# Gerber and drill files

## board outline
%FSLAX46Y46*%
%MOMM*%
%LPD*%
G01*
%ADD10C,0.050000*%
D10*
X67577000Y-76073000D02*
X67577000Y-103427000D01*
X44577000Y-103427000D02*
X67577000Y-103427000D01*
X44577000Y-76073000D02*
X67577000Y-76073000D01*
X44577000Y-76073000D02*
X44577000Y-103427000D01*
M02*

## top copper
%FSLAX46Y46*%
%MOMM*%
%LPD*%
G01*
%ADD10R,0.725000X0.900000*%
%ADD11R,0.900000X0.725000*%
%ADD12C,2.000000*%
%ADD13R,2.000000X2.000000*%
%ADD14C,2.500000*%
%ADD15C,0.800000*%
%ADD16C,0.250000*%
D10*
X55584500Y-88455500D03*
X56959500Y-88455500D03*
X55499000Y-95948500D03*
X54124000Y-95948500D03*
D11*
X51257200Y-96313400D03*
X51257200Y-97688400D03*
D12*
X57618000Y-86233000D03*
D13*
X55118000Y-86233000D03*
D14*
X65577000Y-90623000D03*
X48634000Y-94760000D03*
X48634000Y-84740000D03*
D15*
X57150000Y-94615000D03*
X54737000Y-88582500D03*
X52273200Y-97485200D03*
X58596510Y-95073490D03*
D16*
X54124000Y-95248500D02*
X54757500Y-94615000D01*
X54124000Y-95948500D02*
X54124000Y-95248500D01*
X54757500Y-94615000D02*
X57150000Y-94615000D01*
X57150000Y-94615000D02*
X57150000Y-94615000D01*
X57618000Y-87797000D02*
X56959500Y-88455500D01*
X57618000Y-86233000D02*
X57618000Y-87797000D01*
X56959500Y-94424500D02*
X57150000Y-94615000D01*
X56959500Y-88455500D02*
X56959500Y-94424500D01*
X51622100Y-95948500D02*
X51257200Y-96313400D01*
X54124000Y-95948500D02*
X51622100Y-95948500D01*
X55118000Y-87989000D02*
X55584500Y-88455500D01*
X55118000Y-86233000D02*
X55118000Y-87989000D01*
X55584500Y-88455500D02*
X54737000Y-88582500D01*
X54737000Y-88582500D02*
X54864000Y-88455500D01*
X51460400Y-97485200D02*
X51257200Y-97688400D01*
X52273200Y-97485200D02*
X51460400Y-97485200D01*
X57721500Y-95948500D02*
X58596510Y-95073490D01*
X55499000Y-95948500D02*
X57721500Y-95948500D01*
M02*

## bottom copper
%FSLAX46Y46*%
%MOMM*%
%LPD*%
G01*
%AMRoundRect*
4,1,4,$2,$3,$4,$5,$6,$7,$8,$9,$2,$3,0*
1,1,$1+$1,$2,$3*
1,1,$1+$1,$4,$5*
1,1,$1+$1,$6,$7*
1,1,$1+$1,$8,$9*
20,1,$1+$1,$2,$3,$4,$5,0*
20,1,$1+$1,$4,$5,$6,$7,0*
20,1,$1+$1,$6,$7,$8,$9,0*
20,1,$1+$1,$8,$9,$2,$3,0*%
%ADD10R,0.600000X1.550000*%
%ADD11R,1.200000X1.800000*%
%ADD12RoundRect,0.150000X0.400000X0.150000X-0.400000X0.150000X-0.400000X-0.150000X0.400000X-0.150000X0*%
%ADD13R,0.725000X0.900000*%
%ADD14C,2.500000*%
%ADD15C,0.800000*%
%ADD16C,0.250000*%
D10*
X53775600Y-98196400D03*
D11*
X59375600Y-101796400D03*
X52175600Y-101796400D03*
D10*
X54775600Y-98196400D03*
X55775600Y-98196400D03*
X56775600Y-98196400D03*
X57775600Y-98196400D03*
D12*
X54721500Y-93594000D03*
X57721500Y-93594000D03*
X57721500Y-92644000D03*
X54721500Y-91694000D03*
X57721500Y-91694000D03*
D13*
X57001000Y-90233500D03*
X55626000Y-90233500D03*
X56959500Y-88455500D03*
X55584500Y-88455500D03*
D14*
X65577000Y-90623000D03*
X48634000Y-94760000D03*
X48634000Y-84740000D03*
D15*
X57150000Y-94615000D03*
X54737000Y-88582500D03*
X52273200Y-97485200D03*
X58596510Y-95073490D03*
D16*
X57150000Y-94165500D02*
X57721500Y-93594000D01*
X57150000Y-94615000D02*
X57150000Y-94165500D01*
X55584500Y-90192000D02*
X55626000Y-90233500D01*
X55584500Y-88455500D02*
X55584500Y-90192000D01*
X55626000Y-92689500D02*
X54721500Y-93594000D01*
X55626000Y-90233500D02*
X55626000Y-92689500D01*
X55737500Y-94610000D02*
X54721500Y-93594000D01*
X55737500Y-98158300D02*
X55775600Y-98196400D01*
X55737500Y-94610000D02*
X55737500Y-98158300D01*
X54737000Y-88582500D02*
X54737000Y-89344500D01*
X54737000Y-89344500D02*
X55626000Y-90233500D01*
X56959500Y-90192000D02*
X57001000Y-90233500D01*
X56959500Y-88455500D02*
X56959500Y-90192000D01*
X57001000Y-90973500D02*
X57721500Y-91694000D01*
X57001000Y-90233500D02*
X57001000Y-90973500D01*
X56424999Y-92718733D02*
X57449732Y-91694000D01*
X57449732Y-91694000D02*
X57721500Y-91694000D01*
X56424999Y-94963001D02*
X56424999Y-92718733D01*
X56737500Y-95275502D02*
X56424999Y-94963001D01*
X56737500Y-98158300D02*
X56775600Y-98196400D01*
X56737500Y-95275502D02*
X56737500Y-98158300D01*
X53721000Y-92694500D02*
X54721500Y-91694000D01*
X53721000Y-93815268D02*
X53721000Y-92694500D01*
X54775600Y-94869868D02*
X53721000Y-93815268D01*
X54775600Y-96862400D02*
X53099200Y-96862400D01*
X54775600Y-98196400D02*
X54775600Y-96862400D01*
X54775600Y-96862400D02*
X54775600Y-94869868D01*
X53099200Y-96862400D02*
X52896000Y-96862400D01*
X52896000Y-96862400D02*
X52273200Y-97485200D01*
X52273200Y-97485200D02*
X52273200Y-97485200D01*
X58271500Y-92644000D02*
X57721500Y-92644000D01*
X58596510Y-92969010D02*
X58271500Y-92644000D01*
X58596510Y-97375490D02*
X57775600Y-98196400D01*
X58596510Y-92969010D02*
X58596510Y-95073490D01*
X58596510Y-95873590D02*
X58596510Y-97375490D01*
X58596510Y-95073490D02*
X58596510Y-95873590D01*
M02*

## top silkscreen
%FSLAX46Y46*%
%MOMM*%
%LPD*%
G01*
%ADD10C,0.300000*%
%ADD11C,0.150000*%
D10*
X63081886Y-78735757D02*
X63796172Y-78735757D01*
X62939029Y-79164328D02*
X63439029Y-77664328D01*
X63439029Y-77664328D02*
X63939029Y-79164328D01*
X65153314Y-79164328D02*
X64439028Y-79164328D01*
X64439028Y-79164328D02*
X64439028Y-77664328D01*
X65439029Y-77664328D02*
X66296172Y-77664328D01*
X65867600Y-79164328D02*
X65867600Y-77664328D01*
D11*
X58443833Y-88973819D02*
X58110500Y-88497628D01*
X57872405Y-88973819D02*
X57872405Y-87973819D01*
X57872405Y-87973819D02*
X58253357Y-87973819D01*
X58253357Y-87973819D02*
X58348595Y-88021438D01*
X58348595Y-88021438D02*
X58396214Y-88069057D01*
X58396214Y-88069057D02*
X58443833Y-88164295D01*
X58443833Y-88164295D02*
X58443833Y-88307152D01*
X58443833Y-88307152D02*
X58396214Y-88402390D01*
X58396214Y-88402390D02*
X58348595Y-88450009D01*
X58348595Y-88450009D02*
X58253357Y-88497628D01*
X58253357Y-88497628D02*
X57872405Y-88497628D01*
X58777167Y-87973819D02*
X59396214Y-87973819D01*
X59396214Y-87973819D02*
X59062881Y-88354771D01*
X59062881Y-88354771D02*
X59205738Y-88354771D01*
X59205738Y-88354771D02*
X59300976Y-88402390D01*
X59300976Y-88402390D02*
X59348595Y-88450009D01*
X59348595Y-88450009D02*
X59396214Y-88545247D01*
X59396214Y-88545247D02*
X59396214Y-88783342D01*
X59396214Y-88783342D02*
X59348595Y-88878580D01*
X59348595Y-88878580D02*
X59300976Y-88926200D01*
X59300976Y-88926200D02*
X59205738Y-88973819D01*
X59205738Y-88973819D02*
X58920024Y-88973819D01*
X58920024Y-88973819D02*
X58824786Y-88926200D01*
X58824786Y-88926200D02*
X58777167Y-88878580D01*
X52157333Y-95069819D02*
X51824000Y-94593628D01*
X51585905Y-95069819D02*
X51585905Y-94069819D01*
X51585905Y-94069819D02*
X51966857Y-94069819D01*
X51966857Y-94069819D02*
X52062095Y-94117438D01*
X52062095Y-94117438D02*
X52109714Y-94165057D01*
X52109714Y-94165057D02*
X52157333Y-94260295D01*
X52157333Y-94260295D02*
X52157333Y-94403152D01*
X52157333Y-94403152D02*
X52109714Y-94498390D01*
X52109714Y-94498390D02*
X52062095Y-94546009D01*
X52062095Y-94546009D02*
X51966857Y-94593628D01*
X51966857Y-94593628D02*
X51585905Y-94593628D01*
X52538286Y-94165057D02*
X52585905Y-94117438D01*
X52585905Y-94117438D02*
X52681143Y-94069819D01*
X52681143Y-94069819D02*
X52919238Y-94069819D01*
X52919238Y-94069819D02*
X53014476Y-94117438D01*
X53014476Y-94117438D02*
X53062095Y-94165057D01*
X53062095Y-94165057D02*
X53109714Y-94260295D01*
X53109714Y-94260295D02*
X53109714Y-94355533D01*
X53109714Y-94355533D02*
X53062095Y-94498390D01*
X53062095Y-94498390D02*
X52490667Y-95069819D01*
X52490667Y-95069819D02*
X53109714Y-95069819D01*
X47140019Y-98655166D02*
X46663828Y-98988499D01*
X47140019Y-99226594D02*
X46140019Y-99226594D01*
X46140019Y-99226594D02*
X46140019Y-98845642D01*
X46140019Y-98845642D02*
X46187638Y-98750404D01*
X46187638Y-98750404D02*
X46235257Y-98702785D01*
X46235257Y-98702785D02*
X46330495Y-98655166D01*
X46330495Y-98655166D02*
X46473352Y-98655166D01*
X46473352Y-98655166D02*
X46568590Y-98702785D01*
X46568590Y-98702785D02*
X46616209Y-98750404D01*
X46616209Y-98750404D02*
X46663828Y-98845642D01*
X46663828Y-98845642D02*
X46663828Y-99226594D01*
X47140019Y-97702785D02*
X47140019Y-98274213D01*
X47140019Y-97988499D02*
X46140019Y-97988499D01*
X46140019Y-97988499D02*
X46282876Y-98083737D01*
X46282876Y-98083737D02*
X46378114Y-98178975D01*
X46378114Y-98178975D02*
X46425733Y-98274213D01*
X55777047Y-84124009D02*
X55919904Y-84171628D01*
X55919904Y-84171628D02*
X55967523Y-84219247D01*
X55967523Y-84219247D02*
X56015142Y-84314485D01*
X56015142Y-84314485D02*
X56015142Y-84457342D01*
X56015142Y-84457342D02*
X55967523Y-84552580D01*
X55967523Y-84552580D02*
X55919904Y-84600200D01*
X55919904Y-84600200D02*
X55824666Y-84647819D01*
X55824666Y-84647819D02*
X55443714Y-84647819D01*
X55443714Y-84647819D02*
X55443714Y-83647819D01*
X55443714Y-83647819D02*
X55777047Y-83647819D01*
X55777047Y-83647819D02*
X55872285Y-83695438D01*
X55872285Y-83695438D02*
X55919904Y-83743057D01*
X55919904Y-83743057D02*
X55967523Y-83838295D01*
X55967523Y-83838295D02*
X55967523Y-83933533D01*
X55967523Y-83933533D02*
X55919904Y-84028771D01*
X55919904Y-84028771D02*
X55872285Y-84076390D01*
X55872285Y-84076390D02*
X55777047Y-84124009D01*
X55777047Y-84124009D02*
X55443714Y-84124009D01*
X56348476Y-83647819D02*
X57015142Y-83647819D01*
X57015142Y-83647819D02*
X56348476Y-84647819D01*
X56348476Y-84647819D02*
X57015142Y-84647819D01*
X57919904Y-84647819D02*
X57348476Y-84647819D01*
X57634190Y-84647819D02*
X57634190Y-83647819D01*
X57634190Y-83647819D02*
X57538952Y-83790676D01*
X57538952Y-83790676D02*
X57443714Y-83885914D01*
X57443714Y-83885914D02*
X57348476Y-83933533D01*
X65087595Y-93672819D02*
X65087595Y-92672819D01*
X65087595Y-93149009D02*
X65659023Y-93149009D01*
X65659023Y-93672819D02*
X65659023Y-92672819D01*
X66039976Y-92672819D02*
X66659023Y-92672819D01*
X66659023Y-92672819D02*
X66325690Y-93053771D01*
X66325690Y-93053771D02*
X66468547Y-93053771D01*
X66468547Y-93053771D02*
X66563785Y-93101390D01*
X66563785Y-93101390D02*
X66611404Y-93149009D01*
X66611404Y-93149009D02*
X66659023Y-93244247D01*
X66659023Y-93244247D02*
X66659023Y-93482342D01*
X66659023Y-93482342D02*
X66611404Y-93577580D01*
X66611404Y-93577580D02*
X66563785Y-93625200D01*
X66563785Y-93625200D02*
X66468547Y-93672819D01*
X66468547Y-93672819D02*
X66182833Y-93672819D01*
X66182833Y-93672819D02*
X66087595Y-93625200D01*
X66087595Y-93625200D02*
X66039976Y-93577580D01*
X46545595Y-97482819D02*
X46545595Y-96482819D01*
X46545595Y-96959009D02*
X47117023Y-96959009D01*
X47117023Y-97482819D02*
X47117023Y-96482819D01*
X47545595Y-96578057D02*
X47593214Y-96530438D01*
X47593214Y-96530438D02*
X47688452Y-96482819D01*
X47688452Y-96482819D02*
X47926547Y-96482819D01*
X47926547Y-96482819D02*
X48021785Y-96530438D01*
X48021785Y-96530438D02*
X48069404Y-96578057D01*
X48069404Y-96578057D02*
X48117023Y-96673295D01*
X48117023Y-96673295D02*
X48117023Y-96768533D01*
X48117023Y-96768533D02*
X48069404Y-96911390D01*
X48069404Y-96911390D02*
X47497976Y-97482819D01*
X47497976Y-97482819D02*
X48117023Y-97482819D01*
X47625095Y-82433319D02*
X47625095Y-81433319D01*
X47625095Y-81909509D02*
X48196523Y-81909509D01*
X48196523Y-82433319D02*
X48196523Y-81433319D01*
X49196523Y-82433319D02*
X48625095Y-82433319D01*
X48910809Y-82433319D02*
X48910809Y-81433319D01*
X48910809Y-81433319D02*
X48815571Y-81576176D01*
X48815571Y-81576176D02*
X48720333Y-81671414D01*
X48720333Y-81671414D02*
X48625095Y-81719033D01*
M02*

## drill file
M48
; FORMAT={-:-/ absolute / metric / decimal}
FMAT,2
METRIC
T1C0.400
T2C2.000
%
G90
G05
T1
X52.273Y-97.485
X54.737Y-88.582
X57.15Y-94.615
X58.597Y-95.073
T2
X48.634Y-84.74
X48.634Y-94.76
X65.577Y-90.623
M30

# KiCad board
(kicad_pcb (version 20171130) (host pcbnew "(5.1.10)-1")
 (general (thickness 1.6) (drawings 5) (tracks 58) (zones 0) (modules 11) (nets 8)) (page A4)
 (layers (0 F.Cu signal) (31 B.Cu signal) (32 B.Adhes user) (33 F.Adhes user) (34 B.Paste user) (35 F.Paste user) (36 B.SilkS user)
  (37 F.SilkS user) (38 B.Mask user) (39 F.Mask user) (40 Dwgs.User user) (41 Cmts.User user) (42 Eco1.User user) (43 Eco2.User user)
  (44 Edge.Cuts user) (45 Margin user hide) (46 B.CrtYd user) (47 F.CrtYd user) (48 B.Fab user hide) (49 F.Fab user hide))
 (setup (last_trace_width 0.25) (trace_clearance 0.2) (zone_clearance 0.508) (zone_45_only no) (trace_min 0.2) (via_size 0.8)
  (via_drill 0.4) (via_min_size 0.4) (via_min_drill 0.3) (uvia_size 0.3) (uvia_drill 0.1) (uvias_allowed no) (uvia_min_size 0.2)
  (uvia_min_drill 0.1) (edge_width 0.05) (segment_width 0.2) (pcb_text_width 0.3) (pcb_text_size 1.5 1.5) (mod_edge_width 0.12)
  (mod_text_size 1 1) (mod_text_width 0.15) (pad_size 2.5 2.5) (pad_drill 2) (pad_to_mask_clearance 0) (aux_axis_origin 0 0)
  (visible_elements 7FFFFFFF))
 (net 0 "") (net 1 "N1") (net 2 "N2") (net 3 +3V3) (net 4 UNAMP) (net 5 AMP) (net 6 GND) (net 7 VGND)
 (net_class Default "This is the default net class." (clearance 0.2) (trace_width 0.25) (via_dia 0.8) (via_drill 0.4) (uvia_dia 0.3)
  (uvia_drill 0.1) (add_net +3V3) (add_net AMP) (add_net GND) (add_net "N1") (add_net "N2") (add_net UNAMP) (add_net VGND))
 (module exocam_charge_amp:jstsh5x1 (layer B.Cu) (at 54.9656 95.6564 180)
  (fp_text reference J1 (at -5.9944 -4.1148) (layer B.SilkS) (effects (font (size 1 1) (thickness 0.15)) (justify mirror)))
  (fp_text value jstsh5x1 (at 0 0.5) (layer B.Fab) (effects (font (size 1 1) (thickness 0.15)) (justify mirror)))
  (pad 5 smd rect (at 1.19 -2.54 180) (size 0.6 1.55) (layers B.Cu B.Paste B.Mask) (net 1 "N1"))
  (pad 6 smd rect (at -4.41 -6.14 180) (size 1.2 1.8) (layers B.Cu B.Paste B.Mask) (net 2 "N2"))
  (pad 6 smd rect (at 2.79 -6.14 180) (size 1.2 1.8) (layers B.Cu B.Paste B.Mask) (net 2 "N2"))
  (pad 4 smd rect (at 0.19 -2.54 180) (size 0.6 1.55) (layers B.Cu B.Paste B.Mask) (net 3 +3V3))
  (pad 3 smd rect (at -0.81 -2.54 180) (size 0.6 1.55) (layers B.Cu B.Paste B.Mask) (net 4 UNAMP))
  (pad 2 smd rect (at -1.81 -2.54 180) (size 0.6 1.55) (layers B.Cu B.Paste B.Mask) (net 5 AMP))
  (pad 1 smd rect (at -2.81 -2.54 180) (size 0.6 1.55) (layers B.Cu B.Paste B.Mask) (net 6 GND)))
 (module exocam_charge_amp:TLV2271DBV (layer B.Cu) (at 56.4515 89.154 180)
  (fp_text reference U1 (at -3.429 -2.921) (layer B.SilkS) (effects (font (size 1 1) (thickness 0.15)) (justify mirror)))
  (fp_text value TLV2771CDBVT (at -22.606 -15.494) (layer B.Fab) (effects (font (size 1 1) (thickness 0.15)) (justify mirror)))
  (pad 4 smd roundrect (at 1.73 -4.44 180) (size 1.1 0.6) (layers B.Cu B.Paste B.Mask) (roundrect_rratio 0.25) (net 4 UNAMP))
  (pad 3 smd roundrect (at -1.27 -4.44 180) (size 1.1 0.6) (layers B.Cu B.Paste B.Mask) (roundrect_rratio 0.25) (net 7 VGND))
  (pad 2 smd roundrect (at -1.27 -3.49 180) (size 1.1 0.6) (layers B.Cu B.Paste B.Mask) (roundrect_rratio 0.25) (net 6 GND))
  (pad 5 smd roundrect (at 1.73 -2.54 180) (size 1.1 0.6) (layers B.Cu B.Paste B.Mask) (roundrect_rratio 0.25) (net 3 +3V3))
  (pad 1 smd roundrect (at -1.27 -2.54 180) (size 1.1 0.6) (layers B.Cu B.Paste B.Mask) (roundrect_rratio 0.25) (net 5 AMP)))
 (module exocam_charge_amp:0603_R (layer B.Cu) (at 56.896 92.7735)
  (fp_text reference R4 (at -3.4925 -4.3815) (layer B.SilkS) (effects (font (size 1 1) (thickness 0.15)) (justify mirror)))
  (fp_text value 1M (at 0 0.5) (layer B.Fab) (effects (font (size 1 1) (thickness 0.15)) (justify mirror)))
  (pad 2 smd rect (at 0.105 -2.54) (size 0.725 0.9) (layers B.Cu B.Paste B.Mask) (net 5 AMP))
  (pad 1 smd rect (at -1.27 -2.54) (size 0.725 0.9) (layers B.Cu B.Paste B.Mask) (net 4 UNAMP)))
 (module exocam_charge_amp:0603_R (layer F.Cu) (at 55.6895 90.9955 180)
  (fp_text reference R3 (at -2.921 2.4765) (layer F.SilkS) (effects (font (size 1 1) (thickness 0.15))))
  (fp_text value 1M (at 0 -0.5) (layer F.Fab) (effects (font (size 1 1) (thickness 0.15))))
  (pad 2 smd rect (at 0.105 2.54 180) (size 0.725 0.9) (layers F.Cu F.Paste F.Mask) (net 4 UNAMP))
  (pad 1 smd rect (at -1.27 2.54 180) (size 0.725 0.9) (layers F.Cu F.Paste F.Mask) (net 7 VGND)))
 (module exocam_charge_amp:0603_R (layer F.Cu) (at 55.394 93.4085)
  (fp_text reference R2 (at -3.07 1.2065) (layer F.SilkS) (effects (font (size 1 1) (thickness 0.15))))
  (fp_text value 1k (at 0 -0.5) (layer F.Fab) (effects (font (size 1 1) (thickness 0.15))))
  (pad 2 smd rect (at 0.105 2.54) (size 0.725 0.9) (layers F.Cu F.Paste F.Mask) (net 6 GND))
  (pad 1 smd rect (at -1.27 2.54) (size 0.725 0.9) (layers F.Cu F.Paste F.Mask) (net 7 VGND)))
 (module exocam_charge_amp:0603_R (layer F.Cu) (at 48.7172 96.4184 90)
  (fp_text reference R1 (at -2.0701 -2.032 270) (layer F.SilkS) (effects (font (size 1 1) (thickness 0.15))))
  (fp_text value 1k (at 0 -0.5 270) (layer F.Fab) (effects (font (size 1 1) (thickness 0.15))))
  (pad 2 smd rect (at 0.105 2.54 90) (size 0.725 0.9) (layers F.Cu F.Paste F.Mask) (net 7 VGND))
  (pad 1 smd rect (at -1.27 2.54 90) (size 0.725 0.9) (layers F.Cu F.Paste F.Mask) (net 3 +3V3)))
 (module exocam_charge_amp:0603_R (layer B.Cu) (at 56.8545 90.9955)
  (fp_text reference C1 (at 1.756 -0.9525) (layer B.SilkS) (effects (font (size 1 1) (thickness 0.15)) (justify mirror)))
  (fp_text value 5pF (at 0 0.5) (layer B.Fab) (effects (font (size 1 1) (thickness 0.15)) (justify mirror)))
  (pad 2 smd rect (at 0.105 -2.54) (size 0.725 0.9) (layers B.Cu B.Paste B.Mask) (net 5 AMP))
  (pad 1 smd rect (at -1.27 -2.54) (size 0.725 0.9) (layers B.Cu B.Paste B.Mask) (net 4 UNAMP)))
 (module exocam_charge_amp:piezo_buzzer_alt (layer F.Cu) (at 56.658 83.693)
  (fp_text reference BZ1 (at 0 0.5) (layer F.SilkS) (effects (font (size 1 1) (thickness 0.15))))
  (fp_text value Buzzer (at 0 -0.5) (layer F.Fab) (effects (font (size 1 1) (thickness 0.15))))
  (pad 2 smd circle (at 0.96 2.54) (size 2 2) (layers F.Cu F.Paste F.Mask) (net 7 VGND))
  (pad 1 smd rect (at -1.54 2.54) (size 2 2) (layers F.Cu F.Paste F.Mask) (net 4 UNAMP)))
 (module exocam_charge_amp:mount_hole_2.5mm (layer F.Cu) (at 60.1815 91.44)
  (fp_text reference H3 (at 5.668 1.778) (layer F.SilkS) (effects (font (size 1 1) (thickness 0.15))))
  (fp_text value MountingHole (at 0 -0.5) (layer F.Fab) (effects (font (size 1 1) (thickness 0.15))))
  (pad 1 thru_hole circle (at 5.3955 -0.817) (size 2.5 2.5) (drill 2) (layers *.Cu *.Mask)))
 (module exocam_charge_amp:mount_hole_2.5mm (layer F.Cu) (at 48.7045 94.9325)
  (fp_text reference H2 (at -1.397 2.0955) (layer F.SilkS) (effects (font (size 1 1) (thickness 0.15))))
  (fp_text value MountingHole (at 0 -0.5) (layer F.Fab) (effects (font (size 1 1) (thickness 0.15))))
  (pad 1 thru_hole circle (at -0.0705 -0.1725) (size 2.5 2.5) (drill 2) (layers *.Cu *.Mask)))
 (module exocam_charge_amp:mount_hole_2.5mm (layer F.Cu) (at 48.641 75.565)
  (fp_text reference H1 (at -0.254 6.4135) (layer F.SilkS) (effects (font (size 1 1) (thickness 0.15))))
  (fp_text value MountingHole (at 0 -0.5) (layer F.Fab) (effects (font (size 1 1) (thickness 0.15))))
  (pad 1 thru_hole circle (at -0.007 9.175) (size 2.5 2.5) (drill 2) (layers *.Cu *.Mask)))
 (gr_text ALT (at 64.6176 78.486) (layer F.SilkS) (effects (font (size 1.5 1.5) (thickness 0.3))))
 (gr_line (start 67.577 76.073) (end 67.577 103.427) (layer Edge.Cuts) (width 0.05))
 (gr_line (start 44.577 103.427) (end 67.577 103.427) (layer Edge.Cuts) (width 0.05))
 (gr_line (start 44.577 76.073) (end 67.577 76.073) (layer Edge.Cuts) (width 0.05))
 (gr_line (start 44.577 76.073) (end 44.577 103.427) (layer Edge.Cuts) (width 0.05))
 (segment (start 54.124 95.2485) (end 54.7575 94.615) (width 0.25) (layer F.Cu) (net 7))
 (segment (start 54.124 95.9485) (end 54.124 95.2485) (width 0.25) (layer F.Cu) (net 7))
 (segment (start 54.7575 94.615) (end 57.15 94.615) (width 0.25) (layer F.Cu) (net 7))
 (segment (start 57.15 94.615) (end 57.15 94.615) (width 0.25) (layer F.Cu) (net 7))
 (via (at 57.15 94.615) (size 0.8) (drill 0.4) (layers F.Cu B.Cu) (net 7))
 (segment (start 57.15 94.1655) (end 57.7215 93.594) (width 0.25) (layer B.Cu) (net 7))
 (segment (start 57.15 94.615) (end 57.15 94.1655) (width 0.25) (layer B.Cu) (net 7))
 (segment (start 57.618 87.797) (end 56.9595 88.4555) (width 0.25) (layer F.Cu) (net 7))
 (segment (start 57.618 86.233) (end 57.618 87.797) (width 0.25) (layer F.Cu) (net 7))
 (segment (start 56.9595 94.4245) (end 57.15 94.615) (width 0.25) (layer F.Cu) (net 7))
 (segment (start 56.9595 88.4555) (end 56.9595 94.4245) (width 0.25) (layer F.Cu) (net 7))
 (segment (start 51.6221 95.9485) (end 51.2572 96.3134) (width 0.25) (layer F.Cu) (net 7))
 (segment (start 54.124 95.9485) (end 51.6221 95.9485) (width 0.25) (layer F.Cu) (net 7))
 (segment (start 55.5845 90.192) (end 55.626 90.2335) (width 0.25) (layer B.Cu) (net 4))
 (segment (start 55.5845 88.4555) (end 55.5845 90.192) (width 0.25) (layer B.Cu) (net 4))
 (segment (start 55.626 92.6895) (end 54.7215 93.594) (width 0.25) (layer B.Cu) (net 4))
 (segment (start 55.626 90.2335) (end 55.626 92.6895) (width 0.25) (layer B.Cu) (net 4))
 (segment (start 55.7375 94.61) (end 54.7215 93.594) (width 0.25) (layer B.Cu) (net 4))
 (segment (start 55.118 87.989) (end 55.5845 88.4555) (width 0.25) (layer F.Cu) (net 4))
 (segment (start 55.118 86.233) (end 55.118 87.989) (width 0.25) (layer F.Cu) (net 4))
 (segment (start 55.5845 88.4555) (end 54.737 88.5825) (width 0.25) (layer F.Cu) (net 4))
 (segment (start 54.737 88.5825) (end 54.864 88.4555) (width 0.25) (layer F.Cu) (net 4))
 (via (at 54.737 88.5825) (size 0.8) (drill 0.4) (layers F.Cu B.Cu) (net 4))
 (segment (start 55.7375 98.1583) (end 55.7756 98.1964) (width 0.25) (layer B.Cu) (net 4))
 (segment (start 55.7375 94.61) (end 55.7375 98.1583) (width 0.25) (layer B.Cu) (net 4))
 (segment (start 54.737 88.5825) (end 54.737 89.3445) (width 0.25) (layer B.Cu) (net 4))
 (segment (start 54.737 89.3445) (end 55.626 90.2335) (width 0.25) (layer B.Cu) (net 4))
 (segment (start 56.9595 90.192) (end 57.001 90.2335) (width 0.25) (layer B.Cu) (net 5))
 (segment (start 56.9595 88.4555) (end 56.9595 90.192) (width 0.25) (layer B.Cu) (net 5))
 (segment (start 57.001 90.9735) (end 57.7215 91.694) (width 0.25) (layer B.Cu) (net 5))
 (segment (start 57.001 90.2335) (end 57.001 90.9735) (width 0.25) (layer B.Cu) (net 5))
 (segment (start 56.424999 92.718733) (end 57.449732 91.694) (width 0.25) (layer B.Cu) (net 5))
 (segment (start 57.449732 91.694) (end 57.7215 91.694) (width 0.25) (layer B.Cu) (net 5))
 (segment (start 56.424999 94.963001) (end 56.424999 92.718733) (width 0.25) (layer B.Cu) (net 5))
 (segment (start 56.7375 95.275502) (end 56.424999 94.963001) (width 0.25) (layer B.Cu) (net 5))
 (segment (start 56.7375 98.1583) (end 56.7756 98.1964) (width 0.25) (layer B.Cu) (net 5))
 (segment (start 56.7375 95.275502) (end 56.7375 98.1583) (width 0.25) (layer B.Cu) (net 5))
 (segment (start 53.721 92.6945) (end 54.7215 91.694) (width 0.25) (layer B.Cu) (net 3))
 (segment (start 53.721 93.815268) (end 53.721 92.6945) (width 0.25) (layer B.Cu) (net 3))
 (segment (start 54.7756 94.869868) (end 53.721 93.815268) (width 0.25) (layer B.Cu) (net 3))
 (segment (start 54.7756 96.8624) (end 53.0992 96.8624) (width 0.25) (layer B.Cu) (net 3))
 (segment (start 54.7756 98.1964) (end 54.7756 96.8624) (width 0.25) (layer B.Cu) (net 3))
 (segment (start 54.7756 96.8624) (end 54.7756 94.869868) (width 0.25) (layer B.Cu) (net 3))
 (segment (start 53.0992 96.8624) (end 52.896 96.8624) (width 0.25) (layer B.Cu) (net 3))
 (segment (start 52.896 96.8624) (end 52.2732 97.4852) (width 0.25) (layer B.Cu) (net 3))
 (segment (start 52.2732 97.4852) (end 52.2732 97.4852) (width 0.25) (layer B.Cu) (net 3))
 (via (at 52.2732 97.4852) (size 0.8) (drill 0.4) (layers F.Cu B.Cu) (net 3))
 (segment (start 51.4604 97.4852) (end 51.2572 97.6884) (width 0.25) (layer F.Cu) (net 3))
 (segment (start 52.2732 97.4852) (end 51.4604 97.4852) (width 0.25) (layer F.Cu) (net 3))
 (segment (start 58.2715 92.644) (end 57.7215 92.644) (width 0.25) (layer B.Cu) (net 6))
 (segment (start 58.59651 92.96901) (end 58.2715 92.644) (width 0.25) (layer B.Cu) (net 6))
 (segment (start 58.59651 97.37549) (end 57.7756 98.1964) (width 0.25) (layer B.Cu) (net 6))
 (segment (start 58.59651 92.96901) (end 58.59651 95.07349) (width 0.25) (layer B.Cu) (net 6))
 (segment (start 58.59651 95.87359) (end 58.59651 97.37549) (width 0.25) (layer B.Cu) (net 6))
 (segment (start 58.59651 95.07349) (end 58.59651 95.87359) (width 0.25) (layer B.Cu) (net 6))
 (via (at 58.59651 95.07349) (size 0.8) (drill 0.4) (layers F.Cu B.Cu) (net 6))
 (segment (start 57.7215 95.9485) (end 58.59651 95.07349) (width 0.25) (layer F.Cu) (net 6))
 (segment (start 55.499 95.9485) (end 57.7215 95.9485) (width 0.25) (layer F.Cu) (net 6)))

